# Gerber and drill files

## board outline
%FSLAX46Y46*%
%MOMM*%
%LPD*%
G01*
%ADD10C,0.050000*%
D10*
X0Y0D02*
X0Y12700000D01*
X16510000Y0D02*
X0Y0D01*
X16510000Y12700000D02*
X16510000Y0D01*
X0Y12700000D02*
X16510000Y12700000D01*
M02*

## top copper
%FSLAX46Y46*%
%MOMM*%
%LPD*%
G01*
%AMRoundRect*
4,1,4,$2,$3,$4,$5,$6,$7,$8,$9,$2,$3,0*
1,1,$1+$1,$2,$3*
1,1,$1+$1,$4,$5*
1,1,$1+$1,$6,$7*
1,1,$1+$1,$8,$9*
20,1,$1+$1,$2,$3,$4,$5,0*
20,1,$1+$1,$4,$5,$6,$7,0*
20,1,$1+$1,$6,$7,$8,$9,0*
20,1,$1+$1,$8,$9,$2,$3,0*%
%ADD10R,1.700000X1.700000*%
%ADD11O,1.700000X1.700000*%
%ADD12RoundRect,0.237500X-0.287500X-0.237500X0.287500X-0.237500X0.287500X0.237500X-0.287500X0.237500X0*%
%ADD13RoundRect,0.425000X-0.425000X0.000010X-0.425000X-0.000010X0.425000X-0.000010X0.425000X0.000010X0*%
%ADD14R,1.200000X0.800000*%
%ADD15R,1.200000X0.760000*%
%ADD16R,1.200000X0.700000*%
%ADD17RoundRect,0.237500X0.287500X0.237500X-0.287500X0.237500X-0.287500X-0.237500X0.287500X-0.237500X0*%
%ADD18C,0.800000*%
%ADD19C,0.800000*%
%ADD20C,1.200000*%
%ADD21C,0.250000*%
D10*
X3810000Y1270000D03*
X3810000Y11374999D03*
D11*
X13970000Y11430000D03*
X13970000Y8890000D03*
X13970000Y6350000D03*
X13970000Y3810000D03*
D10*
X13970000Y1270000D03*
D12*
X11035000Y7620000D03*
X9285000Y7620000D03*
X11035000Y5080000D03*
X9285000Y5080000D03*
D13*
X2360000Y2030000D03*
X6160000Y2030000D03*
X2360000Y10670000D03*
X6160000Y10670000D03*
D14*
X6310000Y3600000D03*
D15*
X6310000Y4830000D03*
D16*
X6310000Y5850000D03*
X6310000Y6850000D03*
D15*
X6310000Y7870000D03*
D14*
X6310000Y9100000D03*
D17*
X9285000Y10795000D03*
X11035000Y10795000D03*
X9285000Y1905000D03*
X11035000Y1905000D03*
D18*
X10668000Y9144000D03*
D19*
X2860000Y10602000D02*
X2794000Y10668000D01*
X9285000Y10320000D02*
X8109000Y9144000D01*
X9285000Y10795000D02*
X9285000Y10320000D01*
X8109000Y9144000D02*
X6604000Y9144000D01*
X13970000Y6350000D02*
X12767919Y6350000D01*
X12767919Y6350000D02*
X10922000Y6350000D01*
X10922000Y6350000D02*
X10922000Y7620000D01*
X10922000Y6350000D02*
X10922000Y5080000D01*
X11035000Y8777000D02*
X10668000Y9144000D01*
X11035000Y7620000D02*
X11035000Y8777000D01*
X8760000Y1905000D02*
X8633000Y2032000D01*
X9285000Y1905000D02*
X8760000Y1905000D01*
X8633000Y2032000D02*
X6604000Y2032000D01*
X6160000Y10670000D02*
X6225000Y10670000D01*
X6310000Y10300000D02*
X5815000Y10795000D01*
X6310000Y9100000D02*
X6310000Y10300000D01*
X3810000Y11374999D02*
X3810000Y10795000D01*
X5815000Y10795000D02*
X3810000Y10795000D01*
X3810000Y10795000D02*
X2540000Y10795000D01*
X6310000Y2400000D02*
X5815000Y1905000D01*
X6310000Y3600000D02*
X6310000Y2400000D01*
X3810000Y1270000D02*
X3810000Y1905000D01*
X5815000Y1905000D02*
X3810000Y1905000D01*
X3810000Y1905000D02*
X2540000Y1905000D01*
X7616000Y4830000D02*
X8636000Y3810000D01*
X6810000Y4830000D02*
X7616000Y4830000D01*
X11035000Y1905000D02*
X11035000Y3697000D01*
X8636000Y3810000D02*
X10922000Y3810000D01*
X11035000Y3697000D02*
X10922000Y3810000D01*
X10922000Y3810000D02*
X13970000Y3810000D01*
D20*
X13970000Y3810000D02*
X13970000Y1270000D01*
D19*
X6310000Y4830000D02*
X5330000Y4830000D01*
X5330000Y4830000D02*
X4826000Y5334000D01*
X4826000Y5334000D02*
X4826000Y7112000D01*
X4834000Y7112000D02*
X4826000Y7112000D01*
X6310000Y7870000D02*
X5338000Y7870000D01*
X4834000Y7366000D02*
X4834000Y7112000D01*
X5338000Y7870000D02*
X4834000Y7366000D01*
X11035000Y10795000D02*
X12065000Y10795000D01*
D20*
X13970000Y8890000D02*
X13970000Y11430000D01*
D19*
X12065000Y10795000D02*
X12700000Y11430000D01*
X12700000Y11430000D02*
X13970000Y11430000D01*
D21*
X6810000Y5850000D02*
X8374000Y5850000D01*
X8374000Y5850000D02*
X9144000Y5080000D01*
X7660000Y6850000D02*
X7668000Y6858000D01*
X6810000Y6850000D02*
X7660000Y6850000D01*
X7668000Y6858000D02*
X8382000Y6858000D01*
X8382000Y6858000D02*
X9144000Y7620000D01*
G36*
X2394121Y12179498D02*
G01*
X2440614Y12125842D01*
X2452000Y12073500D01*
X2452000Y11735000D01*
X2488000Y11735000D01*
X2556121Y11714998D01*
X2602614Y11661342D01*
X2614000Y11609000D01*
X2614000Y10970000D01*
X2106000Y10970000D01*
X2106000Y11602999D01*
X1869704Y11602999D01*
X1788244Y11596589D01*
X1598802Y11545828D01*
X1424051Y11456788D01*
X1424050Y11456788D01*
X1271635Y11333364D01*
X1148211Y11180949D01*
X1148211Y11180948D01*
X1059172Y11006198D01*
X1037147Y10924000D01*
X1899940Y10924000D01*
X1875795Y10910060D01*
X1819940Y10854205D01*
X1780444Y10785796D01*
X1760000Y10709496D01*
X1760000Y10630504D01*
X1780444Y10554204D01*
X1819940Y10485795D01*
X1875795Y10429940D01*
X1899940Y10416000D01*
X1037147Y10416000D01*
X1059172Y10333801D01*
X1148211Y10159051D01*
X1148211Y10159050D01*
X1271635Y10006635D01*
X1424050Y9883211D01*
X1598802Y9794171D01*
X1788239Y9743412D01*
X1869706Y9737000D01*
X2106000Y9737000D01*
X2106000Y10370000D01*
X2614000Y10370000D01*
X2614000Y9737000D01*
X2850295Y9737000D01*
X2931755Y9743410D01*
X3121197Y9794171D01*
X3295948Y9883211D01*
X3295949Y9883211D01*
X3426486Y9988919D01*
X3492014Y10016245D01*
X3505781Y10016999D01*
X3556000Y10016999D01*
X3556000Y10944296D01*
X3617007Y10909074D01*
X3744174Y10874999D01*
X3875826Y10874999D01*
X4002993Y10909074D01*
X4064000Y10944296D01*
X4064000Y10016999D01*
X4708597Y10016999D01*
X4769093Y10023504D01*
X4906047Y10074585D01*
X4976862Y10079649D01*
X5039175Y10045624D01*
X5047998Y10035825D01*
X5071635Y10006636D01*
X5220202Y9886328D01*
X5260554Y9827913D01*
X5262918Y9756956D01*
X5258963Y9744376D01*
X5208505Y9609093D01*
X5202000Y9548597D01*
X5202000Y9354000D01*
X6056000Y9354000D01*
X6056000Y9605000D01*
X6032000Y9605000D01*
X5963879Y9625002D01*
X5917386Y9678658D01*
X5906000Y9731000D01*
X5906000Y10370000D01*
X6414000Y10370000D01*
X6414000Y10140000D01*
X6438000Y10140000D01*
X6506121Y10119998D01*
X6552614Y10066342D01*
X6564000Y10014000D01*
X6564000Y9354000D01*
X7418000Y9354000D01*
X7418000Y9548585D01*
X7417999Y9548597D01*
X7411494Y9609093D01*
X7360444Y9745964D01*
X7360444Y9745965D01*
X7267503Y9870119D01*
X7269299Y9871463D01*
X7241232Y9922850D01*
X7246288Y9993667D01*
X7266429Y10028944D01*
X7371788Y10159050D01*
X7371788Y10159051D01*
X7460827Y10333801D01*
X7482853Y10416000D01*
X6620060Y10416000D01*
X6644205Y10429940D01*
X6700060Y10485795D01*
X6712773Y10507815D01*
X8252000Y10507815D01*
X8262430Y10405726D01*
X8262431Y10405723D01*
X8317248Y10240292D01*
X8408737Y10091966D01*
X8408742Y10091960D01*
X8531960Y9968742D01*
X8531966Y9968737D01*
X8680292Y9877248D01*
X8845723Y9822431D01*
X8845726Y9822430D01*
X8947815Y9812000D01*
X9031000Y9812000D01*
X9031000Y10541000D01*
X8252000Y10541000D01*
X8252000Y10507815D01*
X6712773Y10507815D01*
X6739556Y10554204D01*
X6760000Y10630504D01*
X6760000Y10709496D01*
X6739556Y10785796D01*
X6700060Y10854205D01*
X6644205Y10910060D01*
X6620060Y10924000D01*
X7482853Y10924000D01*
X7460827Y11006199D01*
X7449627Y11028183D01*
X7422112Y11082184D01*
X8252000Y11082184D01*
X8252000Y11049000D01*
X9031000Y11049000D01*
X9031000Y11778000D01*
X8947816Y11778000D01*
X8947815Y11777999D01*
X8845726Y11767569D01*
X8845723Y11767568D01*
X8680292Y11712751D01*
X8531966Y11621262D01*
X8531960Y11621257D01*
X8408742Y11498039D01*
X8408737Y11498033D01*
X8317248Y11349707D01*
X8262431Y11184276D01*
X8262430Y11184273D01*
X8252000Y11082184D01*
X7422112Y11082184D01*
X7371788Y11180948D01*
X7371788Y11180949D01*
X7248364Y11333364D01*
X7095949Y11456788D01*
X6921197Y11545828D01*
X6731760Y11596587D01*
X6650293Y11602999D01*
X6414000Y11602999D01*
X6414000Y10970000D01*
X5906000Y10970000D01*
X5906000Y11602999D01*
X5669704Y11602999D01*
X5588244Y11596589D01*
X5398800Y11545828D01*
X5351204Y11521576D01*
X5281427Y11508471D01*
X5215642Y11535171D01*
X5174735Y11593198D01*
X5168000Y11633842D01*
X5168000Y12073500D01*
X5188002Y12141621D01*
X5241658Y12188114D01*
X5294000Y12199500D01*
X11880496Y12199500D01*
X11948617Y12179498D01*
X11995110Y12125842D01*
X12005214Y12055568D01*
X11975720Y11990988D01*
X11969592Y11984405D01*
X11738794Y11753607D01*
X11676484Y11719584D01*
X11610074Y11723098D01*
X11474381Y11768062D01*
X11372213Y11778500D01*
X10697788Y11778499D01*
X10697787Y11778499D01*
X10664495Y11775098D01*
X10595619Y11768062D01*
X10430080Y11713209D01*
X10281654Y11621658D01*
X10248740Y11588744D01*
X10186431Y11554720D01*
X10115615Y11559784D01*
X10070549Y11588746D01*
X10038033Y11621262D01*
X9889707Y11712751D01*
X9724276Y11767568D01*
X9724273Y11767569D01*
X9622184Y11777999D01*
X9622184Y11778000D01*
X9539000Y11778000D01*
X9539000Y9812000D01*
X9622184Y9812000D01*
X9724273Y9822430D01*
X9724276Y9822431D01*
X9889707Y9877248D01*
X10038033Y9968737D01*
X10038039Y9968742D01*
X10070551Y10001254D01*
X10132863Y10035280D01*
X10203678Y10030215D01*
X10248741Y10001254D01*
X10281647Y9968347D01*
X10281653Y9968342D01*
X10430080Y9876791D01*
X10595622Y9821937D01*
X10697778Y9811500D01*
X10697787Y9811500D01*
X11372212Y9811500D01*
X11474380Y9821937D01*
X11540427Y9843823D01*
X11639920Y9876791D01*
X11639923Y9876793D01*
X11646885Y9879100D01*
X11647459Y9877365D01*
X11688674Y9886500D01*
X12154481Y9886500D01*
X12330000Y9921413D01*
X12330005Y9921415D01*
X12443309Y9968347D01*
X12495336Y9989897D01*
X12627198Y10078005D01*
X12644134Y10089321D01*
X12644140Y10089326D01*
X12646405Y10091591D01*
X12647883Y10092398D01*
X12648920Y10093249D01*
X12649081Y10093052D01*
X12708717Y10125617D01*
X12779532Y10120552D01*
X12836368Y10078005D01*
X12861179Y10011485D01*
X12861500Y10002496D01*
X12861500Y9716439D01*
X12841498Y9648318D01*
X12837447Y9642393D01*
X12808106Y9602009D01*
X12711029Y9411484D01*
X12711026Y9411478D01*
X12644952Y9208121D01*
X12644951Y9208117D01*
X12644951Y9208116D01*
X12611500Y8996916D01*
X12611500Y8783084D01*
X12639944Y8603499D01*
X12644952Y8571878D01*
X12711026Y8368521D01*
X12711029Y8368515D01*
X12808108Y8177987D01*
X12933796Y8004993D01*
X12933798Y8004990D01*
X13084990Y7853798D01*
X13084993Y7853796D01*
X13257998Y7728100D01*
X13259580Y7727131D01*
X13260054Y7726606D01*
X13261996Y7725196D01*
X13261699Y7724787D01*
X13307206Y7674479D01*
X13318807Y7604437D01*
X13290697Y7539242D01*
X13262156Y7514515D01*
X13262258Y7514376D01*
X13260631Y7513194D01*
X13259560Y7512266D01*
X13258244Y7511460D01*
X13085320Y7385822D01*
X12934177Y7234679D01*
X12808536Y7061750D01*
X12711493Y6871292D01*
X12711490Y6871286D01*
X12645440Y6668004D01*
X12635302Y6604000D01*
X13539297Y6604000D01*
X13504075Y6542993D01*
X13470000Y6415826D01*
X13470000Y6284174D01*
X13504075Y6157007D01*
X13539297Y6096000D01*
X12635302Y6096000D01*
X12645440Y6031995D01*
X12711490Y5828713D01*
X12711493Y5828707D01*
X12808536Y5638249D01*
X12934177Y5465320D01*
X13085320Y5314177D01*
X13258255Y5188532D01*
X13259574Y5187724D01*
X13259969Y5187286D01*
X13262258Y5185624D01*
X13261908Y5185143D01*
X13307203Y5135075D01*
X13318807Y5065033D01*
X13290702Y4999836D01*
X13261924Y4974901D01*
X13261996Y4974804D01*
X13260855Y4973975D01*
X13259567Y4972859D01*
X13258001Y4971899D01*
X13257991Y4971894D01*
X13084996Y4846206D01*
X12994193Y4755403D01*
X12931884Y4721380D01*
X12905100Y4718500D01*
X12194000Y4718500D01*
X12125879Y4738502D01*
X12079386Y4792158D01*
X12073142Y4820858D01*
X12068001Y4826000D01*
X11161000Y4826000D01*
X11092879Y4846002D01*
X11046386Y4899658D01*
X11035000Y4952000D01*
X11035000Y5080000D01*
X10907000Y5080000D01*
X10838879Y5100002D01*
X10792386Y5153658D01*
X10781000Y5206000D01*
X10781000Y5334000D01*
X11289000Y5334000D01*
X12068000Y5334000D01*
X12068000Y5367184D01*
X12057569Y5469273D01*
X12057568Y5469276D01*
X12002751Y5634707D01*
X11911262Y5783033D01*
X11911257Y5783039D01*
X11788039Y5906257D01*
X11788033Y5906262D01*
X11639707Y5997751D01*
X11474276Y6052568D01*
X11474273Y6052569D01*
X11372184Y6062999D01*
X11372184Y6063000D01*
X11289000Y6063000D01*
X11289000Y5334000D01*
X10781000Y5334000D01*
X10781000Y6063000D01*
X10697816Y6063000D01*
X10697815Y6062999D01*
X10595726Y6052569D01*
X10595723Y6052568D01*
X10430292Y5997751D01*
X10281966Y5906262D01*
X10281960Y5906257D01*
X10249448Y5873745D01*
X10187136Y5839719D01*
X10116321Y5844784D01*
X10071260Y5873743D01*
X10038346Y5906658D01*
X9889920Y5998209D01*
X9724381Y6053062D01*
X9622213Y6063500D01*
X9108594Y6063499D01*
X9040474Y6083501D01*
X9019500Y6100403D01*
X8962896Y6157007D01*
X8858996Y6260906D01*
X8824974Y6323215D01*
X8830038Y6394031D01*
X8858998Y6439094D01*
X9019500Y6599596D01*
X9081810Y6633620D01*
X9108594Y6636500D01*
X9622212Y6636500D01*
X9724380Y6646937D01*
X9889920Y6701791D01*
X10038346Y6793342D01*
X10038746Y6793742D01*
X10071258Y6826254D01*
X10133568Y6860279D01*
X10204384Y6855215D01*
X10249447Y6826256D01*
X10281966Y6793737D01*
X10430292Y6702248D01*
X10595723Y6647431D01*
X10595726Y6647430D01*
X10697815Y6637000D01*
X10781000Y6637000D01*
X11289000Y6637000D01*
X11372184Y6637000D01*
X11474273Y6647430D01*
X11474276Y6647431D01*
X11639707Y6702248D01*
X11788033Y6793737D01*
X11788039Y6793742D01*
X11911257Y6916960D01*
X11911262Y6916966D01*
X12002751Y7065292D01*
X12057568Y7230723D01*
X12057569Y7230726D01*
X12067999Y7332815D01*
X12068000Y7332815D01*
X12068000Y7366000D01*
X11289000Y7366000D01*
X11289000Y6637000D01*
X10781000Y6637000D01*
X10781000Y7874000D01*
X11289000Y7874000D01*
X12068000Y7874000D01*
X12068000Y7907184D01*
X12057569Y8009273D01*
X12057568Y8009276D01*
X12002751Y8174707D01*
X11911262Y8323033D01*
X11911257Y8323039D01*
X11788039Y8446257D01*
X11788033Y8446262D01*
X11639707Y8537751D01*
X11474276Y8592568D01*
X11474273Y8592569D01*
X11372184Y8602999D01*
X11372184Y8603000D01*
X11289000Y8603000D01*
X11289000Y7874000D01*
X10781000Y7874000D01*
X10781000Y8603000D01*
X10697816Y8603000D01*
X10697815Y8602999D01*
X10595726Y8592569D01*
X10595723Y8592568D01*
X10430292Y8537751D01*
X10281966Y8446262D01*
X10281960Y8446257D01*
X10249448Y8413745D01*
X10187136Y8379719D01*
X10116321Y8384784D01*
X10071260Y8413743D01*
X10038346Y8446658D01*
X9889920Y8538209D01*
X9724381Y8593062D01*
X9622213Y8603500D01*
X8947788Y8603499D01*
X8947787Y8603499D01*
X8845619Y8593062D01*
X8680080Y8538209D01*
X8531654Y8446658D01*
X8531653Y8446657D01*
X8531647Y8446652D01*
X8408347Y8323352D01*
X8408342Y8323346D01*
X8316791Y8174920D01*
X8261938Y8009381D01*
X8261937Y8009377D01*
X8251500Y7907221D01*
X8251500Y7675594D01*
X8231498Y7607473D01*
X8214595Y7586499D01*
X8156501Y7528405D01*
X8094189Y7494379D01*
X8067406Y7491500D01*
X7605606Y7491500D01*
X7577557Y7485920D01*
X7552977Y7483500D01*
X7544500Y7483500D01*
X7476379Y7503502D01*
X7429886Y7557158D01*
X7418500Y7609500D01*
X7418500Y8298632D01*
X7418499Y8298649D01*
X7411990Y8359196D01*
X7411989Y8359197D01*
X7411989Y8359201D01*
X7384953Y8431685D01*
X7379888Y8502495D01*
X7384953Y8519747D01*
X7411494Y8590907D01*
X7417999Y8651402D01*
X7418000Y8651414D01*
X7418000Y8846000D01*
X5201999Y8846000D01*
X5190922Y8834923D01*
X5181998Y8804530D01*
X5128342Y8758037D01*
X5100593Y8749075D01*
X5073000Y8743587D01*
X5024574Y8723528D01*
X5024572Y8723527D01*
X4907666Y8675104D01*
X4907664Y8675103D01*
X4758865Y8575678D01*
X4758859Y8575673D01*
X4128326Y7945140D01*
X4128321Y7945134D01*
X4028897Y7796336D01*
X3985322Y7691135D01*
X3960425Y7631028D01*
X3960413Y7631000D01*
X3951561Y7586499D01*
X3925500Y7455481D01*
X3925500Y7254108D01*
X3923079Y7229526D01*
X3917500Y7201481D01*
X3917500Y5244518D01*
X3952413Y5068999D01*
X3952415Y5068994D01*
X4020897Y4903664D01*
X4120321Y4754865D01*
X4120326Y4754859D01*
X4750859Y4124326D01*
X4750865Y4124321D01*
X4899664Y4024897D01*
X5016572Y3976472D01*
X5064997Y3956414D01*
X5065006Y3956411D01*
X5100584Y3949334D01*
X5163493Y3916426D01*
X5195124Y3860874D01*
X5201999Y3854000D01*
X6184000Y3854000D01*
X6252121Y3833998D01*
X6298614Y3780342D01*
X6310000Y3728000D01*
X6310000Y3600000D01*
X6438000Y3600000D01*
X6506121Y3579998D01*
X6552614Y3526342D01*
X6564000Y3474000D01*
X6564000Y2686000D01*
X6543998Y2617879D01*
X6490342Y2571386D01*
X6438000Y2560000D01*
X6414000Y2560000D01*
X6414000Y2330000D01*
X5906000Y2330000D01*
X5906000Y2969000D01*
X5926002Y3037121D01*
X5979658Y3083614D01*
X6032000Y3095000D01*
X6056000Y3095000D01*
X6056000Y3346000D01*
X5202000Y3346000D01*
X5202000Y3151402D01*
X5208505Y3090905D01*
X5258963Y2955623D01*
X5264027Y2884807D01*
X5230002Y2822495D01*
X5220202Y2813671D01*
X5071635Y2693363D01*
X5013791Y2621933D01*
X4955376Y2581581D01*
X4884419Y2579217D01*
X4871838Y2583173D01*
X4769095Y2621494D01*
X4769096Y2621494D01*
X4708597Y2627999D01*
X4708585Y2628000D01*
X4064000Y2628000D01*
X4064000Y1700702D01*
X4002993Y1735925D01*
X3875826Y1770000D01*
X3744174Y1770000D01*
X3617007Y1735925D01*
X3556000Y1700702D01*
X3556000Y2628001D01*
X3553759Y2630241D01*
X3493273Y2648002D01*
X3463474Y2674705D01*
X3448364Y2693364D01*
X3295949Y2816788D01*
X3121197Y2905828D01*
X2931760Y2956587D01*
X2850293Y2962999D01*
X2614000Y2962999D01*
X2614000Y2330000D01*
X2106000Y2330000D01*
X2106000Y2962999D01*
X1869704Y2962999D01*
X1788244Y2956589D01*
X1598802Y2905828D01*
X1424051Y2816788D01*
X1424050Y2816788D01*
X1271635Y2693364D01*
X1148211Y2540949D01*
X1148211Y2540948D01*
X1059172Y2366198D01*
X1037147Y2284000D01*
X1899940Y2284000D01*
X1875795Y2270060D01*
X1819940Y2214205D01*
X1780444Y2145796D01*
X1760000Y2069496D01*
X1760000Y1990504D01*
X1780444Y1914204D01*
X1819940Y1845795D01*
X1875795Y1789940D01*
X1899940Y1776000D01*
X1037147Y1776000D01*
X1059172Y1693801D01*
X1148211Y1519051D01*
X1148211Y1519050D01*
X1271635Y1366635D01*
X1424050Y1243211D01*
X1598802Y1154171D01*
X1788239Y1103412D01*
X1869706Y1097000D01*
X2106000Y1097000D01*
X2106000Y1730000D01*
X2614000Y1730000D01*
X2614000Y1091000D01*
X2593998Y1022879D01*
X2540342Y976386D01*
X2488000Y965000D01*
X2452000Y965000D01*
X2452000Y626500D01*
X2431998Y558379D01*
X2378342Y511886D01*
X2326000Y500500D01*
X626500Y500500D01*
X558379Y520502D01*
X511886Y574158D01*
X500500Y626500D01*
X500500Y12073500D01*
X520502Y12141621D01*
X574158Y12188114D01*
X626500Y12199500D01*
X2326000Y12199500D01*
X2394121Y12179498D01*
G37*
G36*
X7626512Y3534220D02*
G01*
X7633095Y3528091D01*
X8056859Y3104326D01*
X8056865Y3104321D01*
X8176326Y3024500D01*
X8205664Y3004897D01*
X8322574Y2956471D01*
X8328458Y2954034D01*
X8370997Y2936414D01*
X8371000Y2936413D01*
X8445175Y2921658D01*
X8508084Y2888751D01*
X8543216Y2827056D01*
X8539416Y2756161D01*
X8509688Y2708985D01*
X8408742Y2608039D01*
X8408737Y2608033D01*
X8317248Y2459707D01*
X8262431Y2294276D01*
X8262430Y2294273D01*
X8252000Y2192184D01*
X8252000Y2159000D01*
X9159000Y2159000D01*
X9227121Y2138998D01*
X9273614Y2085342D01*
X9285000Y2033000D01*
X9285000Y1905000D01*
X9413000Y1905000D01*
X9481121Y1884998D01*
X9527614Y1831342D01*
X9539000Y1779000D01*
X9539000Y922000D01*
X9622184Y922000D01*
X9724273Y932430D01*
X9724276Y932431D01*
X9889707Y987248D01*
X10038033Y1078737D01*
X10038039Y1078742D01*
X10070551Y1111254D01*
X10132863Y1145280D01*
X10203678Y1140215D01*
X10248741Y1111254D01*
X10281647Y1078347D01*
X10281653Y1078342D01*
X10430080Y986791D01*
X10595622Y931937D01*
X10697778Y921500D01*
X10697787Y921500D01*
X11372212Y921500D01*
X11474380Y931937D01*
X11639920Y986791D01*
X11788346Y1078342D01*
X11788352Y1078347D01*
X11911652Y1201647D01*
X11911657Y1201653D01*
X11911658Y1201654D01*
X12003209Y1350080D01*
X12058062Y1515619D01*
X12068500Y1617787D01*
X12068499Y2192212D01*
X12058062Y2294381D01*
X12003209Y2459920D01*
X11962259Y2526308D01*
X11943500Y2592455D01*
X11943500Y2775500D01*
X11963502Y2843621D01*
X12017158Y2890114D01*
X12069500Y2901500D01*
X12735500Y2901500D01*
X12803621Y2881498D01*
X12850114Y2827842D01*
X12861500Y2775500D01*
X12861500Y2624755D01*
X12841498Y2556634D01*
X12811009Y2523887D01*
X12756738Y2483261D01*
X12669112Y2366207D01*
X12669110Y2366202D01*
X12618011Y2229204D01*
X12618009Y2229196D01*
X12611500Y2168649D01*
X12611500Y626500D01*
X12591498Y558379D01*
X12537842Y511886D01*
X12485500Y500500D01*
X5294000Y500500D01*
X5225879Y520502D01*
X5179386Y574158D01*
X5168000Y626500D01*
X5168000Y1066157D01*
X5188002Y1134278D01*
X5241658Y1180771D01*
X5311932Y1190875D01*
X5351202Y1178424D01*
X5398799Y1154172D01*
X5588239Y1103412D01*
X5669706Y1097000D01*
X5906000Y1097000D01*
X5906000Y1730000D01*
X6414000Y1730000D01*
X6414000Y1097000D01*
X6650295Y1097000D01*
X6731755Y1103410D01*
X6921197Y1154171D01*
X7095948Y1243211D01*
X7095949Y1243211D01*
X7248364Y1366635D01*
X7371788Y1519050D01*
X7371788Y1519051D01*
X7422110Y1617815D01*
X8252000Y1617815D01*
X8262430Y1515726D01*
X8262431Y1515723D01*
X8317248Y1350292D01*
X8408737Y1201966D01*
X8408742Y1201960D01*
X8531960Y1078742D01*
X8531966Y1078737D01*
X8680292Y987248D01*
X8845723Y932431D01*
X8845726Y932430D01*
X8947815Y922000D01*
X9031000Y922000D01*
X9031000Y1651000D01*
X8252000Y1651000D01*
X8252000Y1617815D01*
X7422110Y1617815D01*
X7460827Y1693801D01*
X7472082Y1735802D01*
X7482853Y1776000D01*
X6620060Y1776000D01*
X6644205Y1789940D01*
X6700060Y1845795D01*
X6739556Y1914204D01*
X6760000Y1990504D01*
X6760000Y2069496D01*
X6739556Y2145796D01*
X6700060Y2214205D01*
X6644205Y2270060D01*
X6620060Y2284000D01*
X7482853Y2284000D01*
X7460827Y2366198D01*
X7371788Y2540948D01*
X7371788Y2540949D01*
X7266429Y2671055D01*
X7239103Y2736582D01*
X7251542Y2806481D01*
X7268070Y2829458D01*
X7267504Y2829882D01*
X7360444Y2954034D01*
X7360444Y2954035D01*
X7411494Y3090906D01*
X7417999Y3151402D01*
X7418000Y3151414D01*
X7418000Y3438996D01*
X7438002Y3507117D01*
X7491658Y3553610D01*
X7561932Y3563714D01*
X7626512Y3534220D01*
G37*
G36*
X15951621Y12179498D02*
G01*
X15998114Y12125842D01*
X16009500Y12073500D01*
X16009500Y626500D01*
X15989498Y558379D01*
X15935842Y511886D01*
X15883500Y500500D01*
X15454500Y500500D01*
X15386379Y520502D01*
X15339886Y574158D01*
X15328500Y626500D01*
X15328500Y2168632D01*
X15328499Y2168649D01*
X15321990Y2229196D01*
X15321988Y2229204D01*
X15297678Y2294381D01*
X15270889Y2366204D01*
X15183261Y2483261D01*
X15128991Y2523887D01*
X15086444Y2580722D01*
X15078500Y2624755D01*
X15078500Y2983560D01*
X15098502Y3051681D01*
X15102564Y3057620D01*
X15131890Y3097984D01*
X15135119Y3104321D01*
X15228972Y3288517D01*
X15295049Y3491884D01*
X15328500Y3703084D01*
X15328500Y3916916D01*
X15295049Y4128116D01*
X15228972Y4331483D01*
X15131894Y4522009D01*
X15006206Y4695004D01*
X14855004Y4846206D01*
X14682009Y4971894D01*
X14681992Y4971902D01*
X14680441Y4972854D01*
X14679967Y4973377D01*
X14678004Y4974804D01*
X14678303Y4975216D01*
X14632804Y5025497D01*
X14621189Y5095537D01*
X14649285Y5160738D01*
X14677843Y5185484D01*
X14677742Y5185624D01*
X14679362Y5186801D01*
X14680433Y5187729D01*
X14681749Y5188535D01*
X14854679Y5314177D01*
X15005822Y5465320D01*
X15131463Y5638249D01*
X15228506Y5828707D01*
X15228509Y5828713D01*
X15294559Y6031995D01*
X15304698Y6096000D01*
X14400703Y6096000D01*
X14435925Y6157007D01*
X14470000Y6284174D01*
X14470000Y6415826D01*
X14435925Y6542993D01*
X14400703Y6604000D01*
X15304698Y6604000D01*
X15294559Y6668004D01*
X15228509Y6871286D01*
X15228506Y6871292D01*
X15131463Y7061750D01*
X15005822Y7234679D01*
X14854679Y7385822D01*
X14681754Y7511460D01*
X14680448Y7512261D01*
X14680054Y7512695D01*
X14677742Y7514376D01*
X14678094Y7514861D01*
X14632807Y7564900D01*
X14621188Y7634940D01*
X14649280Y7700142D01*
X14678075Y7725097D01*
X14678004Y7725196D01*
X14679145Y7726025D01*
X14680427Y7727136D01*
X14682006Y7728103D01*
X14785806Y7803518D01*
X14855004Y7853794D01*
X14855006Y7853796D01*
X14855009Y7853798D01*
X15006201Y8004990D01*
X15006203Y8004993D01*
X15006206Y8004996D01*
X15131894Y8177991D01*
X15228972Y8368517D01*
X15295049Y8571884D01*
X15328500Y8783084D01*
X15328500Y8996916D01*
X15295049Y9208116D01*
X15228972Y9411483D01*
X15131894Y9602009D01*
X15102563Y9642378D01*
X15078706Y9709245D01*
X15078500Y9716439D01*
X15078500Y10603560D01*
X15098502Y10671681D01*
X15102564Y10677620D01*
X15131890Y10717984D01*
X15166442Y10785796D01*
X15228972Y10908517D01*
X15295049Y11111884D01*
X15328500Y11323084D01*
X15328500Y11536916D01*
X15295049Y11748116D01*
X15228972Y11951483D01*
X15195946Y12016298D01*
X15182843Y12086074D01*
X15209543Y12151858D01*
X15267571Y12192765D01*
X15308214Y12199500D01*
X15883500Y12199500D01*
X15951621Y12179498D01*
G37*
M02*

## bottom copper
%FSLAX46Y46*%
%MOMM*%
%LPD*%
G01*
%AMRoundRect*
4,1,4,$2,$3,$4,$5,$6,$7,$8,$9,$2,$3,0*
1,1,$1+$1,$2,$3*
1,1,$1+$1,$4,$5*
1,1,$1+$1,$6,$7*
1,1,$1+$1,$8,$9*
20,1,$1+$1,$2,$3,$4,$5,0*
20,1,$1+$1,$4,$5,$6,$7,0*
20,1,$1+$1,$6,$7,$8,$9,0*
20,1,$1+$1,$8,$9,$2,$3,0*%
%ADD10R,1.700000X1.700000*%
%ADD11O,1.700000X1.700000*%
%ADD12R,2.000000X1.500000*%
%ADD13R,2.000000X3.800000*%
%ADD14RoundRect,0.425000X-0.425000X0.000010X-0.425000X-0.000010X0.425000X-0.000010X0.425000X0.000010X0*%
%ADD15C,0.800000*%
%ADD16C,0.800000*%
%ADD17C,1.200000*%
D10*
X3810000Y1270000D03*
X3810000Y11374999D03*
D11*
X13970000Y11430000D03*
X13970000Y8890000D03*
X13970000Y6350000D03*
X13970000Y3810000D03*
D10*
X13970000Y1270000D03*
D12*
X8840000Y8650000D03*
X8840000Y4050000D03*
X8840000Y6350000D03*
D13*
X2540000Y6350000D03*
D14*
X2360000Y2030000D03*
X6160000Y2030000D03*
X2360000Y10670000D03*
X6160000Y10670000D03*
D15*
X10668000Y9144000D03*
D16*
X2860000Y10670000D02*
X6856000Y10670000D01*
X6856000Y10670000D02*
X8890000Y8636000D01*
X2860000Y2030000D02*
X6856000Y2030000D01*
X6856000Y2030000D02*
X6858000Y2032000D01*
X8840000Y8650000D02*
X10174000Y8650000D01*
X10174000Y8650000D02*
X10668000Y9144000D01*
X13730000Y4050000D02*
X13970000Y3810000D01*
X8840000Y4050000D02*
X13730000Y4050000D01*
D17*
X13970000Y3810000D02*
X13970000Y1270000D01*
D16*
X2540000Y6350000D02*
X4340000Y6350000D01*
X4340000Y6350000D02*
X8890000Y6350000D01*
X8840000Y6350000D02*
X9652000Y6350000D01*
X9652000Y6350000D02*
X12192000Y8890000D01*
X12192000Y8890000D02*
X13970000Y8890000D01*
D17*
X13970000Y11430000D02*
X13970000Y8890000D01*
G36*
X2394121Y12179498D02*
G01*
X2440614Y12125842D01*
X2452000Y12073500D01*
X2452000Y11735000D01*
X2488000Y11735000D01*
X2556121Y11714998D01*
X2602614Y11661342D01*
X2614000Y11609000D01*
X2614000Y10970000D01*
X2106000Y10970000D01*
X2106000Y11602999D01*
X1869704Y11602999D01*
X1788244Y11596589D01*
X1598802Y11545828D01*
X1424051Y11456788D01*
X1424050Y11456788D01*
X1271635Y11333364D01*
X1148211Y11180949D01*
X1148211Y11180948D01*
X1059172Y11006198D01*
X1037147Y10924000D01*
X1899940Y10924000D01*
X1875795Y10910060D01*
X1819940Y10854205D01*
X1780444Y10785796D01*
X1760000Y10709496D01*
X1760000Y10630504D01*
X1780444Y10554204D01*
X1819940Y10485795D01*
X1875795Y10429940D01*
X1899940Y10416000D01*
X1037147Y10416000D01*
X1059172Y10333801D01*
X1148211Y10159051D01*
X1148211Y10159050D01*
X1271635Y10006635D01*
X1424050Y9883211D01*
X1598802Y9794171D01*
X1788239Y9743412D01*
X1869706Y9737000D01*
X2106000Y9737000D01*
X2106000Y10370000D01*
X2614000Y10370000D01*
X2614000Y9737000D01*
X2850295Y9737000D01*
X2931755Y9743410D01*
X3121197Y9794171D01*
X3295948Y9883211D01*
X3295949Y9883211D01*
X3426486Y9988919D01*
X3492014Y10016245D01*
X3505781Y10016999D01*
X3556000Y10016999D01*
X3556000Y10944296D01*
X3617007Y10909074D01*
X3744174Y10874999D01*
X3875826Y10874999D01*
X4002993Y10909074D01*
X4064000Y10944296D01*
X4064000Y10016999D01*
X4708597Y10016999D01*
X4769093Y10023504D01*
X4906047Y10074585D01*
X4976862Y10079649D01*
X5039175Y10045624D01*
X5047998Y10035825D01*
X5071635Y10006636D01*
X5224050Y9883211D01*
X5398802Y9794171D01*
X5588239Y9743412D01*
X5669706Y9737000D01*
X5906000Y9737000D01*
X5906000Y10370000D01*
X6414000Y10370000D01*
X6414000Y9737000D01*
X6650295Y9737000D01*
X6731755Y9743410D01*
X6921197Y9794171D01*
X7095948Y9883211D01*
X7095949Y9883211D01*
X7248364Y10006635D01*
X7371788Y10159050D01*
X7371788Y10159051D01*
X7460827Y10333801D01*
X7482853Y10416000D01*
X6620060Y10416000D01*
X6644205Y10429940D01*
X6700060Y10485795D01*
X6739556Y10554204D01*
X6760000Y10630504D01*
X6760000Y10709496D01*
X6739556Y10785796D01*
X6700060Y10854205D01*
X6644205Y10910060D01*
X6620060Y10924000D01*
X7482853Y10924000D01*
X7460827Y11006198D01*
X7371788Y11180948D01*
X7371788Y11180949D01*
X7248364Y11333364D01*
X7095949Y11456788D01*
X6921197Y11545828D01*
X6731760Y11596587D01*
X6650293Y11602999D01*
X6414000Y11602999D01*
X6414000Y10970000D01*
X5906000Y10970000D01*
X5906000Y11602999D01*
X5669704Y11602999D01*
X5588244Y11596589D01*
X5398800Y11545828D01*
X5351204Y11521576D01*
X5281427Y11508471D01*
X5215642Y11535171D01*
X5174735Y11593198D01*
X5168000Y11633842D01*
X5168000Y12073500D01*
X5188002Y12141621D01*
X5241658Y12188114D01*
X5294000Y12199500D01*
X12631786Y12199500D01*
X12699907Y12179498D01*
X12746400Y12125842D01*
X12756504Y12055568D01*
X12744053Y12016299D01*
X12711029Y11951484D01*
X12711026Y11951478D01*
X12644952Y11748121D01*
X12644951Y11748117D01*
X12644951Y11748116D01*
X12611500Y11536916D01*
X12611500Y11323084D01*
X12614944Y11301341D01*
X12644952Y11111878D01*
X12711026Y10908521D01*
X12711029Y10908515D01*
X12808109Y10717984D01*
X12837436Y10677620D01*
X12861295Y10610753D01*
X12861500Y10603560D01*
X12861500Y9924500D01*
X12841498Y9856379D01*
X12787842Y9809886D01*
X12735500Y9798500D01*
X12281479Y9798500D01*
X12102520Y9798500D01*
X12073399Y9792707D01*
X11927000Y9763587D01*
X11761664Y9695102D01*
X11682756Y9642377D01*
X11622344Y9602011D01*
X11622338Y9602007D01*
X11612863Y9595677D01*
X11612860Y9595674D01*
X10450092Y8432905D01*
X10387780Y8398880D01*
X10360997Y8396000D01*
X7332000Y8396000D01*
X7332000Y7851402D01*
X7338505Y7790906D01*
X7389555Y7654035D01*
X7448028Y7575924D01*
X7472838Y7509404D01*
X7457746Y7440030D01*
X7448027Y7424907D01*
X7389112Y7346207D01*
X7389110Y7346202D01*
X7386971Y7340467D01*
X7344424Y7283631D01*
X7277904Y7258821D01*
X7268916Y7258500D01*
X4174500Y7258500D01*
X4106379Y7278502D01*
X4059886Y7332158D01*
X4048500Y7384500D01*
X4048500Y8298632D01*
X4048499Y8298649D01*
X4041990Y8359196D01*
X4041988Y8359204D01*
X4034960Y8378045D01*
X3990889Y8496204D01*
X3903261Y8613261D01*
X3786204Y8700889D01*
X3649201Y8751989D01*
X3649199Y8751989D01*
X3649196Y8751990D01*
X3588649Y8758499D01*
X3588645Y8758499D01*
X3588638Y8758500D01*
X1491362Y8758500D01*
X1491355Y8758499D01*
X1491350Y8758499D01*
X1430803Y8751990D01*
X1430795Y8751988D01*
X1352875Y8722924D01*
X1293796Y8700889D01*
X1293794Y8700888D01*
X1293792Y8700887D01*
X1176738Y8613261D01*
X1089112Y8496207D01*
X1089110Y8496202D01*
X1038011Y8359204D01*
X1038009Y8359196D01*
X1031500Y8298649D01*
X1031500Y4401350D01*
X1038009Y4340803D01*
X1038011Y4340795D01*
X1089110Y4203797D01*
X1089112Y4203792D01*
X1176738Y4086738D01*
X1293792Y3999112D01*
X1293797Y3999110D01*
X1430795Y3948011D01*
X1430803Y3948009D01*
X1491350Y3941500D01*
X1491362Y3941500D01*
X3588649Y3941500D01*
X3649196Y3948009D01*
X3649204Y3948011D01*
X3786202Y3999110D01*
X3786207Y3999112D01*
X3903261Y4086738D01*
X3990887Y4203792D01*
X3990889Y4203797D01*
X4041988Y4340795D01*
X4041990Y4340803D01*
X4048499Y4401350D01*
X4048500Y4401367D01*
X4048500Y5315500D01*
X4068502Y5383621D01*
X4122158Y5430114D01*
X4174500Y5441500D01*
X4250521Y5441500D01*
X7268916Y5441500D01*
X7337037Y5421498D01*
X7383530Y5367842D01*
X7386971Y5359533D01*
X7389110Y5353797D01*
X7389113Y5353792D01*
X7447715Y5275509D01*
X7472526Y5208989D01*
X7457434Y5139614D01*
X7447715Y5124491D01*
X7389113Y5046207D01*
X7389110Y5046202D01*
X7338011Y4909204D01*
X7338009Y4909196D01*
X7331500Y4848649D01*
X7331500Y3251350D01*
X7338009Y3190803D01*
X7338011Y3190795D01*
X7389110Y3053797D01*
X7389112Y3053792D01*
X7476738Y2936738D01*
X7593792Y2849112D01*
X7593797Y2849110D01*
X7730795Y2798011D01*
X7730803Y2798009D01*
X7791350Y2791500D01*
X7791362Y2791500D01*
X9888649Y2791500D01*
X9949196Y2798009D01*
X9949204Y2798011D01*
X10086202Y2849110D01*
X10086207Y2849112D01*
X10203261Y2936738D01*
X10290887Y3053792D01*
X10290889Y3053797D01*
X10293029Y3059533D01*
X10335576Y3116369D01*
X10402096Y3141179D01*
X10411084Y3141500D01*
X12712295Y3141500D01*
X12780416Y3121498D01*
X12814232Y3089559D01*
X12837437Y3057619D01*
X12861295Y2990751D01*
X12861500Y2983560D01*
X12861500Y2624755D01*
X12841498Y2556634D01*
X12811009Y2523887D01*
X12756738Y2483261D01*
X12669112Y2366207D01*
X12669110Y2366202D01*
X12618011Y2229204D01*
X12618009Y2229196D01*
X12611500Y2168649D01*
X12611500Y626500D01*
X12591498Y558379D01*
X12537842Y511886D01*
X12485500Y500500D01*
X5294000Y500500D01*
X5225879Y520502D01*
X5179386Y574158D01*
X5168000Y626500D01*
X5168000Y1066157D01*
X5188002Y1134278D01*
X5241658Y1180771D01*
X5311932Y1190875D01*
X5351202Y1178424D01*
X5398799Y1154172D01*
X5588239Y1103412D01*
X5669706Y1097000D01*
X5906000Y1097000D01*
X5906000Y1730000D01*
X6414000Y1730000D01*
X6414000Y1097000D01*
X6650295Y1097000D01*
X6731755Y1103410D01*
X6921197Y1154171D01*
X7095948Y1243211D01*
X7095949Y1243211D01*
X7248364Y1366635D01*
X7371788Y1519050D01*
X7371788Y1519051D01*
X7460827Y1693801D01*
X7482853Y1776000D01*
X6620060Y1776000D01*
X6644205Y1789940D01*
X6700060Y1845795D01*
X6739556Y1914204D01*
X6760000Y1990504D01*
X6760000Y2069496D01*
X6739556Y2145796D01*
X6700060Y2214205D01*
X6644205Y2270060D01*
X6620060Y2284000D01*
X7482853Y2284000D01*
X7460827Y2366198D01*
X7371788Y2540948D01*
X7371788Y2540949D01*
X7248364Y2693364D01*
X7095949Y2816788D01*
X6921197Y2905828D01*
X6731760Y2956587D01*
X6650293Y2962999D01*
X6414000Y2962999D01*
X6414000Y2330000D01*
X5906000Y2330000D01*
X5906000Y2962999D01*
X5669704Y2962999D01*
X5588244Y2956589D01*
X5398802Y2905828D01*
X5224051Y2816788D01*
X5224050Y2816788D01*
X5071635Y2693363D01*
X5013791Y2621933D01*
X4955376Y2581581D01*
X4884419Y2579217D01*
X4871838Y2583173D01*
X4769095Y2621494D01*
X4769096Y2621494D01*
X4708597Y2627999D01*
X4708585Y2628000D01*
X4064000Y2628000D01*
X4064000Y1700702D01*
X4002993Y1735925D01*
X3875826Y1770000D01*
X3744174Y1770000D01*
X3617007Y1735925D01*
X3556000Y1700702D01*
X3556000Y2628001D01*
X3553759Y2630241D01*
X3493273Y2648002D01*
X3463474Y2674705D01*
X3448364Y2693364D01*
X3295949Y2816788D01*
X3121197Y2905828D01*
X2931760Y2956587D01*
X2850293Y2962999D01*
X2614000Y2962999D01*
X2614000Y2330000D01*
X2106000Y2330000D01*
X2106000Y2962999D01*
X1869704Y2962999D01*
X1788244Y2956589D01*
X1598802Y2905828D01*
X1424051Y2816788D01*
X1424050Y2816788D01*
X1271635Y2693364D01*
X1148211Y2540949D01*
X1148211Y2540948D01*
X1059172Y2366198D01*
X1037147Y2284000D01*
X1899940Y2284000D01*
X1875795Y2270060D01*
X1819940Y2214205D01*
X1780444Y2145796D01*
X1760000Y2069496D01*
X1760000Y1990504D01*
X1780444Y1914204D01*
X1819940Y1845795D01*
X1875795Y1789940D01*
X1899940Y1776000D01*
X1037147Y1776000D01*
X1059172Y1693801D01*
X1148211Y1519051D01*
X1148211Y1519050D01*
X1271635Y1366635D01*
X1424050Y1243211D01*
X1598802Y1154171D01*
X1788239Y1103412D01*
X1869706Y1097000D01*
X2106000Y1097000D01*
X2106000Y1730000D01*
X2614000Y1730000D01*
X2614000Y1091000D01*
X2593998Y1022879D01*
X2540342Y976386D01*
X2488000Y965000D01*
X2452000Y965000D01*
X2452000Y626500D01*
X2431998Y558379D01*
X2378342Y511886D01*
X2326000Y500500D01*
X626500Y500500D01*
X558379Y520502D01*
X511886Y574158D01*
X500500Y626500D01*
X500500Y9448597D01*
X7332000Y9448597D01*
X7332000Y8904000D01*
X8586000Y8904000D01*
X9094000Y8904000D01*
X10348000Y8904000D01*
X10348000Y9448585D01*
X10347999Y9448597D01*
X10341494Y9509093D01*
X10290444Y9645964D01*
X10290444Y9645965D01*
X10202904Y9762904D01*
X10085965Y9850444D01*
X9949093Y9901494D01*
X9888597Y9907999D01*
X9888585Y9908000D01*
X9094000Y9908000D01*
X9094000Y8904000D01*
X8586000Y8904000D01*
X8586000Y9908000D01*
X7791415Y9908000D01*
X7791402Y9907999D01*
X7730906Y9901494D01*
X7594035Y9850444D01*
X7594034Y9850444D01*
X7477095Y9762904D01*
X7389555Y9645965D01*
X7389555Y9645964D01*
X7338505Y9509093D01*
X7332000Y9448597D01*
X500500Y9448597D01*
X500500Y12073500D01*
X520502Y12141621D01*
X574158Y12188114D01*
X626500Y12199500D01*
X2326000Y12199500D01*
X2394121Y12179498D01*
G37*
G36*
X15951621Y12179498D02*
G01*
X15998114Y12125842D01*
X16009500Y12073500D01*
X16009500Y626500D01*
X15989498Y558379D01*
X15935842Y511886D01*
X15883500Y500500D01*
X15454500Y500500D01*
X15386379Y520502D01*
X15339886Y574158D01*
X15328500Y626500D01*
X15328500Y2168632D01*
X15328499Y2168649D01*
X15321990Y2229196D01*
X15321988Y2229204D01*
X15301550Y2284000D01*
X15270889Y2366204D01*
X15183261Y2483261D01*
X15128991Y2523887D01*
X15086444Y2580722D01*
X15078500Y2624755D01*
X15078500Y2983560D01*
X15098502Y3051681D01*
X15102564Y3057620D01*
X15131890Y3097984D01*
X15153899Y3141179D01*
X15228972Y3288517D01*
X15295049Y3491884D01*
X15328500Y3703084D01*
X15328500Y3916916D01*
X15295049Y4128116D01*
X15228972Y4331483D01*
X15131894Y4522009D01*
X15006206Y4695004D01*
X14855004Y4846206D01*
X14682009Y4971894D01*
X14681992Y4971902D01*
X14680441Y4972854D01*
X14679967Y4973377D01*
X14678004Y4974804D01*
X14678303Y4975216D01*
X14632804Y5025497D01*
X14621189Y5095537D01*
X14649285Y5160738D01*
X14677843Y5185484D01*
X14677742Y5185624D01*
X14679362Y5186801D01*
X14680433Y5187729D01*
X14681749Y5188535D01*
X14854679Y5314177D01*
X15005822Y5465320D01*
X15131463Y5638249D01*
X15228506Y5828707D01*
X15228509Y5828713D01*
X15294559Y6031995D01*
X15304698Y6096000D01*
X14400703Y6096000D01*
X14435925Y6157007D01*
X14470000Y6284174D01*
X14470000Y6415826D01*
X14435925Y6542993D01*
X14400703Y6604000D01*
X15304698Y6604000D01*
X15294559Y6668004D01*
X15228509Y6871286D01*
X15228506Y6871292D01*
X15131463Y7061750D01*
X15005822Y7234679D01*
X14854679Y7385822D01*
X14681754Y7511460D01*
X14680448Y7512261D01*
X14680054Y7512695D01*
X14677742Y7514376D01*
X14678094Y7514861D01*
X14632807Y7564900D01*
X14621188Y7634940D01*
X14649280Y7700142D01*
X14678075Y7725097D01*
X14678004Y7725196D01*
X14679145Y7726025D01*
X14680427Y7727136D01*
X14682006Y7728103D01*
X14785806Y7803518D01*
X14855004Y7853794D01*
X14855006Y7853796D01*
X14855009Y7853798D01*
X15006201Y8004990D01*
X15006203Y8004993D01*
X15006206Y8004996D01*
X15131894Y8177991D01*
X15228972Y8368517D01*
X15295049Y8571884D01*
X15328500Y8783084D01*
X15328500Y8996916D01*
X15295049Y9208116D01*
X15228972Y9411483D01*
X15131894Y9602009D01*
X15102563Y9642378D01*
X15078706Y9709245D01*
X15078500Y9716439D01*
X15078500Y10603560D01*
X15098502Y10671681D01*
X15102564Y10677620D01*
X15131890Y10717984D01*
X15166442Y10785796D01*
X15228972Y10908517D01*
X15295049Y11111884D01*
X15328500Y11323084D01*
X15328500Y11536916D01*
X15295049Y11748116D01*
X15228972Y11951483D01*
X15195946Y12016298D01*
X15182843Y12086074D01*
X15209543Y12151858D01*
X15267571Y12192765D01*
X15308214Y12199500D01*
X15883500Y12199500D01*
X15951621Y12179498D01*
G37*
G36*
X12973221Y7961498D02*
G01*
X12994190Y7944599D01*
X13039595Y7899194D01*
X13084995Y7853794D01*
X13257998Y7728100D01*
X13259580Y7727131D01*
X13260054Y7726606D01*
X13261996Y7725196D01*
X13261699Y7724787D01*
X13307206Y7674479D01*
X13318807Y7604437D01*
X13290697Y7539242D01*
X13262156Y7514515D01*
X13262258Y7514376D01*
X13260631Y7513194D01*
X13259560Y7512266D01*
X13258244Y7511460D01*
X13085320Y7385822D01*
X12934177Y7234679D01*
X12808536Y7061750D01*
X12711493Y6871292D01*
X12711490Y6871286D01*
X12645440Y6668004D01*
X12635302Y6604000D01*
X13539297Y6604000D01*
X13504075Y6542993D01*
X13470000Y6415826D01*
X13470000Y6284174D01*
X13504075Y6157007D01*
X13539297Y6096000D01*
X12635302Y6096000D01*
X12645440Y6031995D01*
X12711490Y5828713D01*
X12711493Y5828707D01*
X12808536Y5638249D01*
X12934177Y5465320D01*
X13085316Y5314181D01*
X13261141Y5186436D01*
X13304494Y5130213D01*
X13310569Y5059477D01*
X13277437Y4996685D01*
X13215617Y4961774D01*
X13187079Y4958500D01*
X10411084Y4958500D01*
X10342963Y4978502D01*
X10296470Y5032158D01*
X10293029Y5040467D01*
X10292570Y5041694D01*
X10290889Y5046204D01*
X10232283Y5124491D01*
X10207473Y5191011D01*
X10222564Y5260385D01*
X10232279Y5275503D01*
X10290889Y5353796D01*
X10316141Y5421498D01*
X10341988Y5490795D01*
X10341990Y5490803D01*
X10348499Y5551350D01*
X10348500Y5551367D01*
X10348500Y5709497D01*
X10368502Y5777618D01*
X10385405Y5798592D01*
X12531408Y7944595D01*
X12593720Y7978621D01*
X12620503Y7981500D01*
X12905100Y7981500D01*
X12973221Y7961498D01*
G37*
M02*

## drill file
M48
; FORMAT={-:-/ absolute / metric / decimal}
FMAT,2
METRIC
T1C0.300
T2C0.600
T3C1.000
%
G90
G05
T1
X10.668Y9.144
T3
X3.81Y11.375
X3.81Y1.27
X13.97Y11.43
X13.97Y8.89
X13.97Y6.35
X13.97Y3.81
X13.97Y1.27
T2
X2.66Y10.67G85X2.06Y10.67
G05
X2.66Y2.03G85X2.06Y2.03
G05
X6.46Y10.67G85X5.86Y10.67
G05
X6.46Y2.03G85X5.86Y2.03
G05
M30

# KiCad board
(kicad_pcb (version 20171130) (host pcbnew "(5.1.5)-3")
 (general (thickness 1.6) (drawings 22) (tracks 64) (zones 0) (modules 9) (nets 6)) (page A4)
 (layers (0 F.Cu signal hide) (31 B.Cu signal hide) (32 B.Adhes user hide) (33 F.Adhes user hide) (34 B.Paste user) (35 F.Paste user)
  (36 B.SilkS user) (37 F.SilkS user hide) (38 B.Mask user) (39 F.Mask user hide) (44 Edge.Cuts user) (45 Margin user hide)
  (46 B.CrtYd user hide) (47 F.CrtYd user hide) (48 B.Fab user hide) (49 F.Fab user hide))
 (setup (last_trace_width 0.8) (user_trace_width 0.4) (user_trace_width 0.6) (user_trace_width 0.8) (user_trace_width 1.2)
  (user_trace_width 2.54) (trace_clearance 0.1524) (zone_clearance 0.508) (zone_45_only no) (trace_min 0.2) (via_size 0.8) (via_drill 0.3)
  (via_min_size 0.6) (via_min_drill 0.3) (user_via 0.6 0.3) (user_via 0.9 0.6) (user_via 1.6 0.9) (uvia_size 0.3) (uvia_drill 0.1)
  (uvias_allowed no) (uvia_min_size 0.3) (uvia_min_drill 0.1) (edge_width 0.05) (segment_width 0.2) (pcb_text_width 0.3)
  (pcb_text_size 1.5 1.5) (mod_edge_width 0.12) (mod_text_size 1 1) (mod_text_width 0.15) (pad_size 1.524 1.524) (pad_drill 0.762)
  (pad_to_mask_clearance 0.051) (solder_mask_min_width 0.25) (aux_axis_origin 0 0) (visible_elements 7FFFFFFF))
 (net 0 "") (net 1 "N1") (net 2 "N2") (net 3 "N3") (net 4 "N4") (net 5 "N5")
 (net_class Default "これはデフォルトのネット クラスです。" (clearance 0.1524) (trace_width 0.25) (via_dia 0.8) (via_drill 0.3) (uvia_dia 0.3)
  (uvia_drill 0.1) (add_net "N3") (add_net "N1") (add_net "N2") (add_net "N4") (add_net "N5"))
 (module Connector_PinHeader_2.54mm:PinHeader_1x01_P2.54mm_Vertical (layer F.Cu) (at 3.81 -1.27 180)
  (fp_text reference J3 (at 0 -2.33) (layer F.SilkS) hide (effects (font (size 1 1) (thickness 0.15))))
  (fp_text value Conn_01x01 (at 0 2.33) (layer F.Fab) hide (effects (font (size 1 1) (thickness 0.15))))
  (pad 1 thru_hole rect (at 0 0 180) (size 1.7 1.7) (drill 1) (layers *.Cu *.Mask) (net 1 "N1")))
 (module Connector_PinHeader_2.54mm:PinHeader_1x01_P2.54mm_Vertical (layer F.Cu) (at 3.81 -11.374999)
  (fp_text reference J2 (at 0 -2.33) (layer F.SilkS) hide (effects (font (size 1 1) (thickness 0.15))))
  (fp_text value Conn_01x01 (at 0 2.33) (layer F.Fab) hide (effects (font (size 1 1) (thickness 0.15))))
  (pad 1 thru_hole rect (at 0 0) (size 1.7 1.7) (drill 1) (layers *.Cu *.Mask) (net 1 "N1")))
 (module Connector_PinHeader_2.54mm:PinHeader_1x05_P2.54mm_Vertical (layer F.Cu) (at 13.97 -1.27 180)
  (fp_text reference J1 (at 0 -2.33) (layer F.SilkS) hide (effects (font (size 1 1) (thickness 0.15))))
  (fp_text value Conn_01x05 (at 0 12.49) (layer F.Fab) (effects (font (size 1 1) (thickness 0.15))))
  (pad 5 thru_hole oval (at 0 10.16 180) (size 1.7 1.7) (drill 1) (layers *.Cu *.Mask) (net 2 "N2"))
  (pad 4 thru_hole oval (at 0 7.62 180) (size 1.7 1.7) (drill 1) (layers *.Cu *.Mask) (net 2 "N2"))
  (pad 3 thru_hole oval (at 0 5.08 180) (size 1.7 1.7) (drill 1) (layers *.Cu *.Mask) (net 1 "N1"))
  (pad 2 thru_hole oval (at 0 2.54 180) (size 1.7 1.7) (drill 1) (layers *.Cu *.Mask) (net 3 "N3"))
  (pad 1 thru_hole rect (at 0 0 180) (size 1.7 1.7) (drill 1) (layers *.Cu *.Mask) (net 3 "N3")))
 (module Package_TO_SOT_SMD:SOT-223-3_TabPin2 (layer B.Cu) (at 5.69 -6.35 180)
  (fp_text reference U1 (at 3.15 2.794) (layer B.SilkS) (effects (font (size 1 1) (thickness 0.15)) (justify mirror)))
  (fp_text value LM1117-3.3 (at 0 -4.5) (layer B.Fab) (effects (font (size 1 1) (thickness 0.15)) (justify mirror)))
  (pad 1 smd rect (at -3.15 2.3 180) (size 2 1.5) (layers B.Cu B.Paste B.Mask) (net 1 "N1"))
  (pad 3 smd rect (at -3.15 -2.3 180) (size 2 1.5) (layers B.Cu B.Paste B.Mask) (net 3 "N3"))
  (pad 2 smd rect (at -3.15 0 180) (size 2 1.5) (layers B.Cu B.Paste B.Mask) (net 2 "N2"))
  (pad 2 smd rect (at 3.15 0 180) (size 2 3.8) (layers B.Cu B.Paste B.Mask) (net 2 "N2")))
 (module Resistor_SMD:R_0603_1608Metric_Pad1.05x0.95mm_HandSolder (layer F.Cu) (at 10.16 -7.62)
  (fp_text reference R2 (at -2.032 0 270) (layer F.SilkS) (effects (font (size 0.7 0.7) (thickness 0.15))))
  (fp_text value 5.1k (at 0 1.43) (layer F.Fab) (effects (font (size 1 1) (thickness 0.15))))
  (pad 2 smd roundrect (at 0.875 0) (size 1.05 0.95) (layers F.Cu F.Paste F.Mask) (roundrect_rratio 0.25) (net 1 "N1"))
  (pad 1 smd roundrect (at -0.875 0) (size 1.05 0.95) (layers F.Cu F.Paste F.Mask) (roundrect_rratio 0.25) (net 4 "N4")))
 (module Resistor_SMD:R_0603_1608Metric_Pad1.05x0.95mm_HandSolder (layer F.Cu) (at 10.16 -5.08)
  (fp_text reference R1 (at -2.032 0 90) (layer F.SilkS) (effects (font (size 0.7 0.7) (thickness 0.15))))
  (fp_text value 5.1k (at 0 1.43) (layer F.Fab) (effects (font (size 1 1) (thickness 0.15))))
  (pad 2 smd roundrect (at 0.875 0) (size 1.05 0.95) (layers F.Cu F.Paste F.Mask) (roundrect_rratio 0.25) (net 1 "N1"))
  (pad 1 smd roundrect (at -0.875 0) (size 1.05 0.95) (layers F.Cu F.Paste F.Mask) (roundrect_rratio 0.25) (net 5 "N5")))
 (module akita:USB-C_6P (layer F.Cu) (at 3.31 -6.35 270)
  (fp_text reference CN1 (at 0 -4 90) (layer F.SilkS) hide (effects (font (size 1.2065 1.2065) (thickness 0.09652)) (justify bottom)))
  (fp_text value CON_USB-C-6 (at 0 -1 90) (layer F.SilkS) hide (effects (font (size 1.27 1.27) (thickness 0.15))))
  (pad FG thru_hole roundrect (at 4.32 0.95 270) (size 0.85 1.7) (drill oval 0.6 1.2) (layers *.Cu *.Mask) (roundrect_rratio 0.5)
   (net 1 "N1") (solder_mask_margin 0.1016))
  (pad FG thru_hole roundrect (at 4.32 -2.85 270) (size 0.85 1.7) (drill oval 0.6 1.2) (layers *.Cu *.Mask) (roundrect_rratio 0.5)
   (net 1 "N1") (solder_mask_margin 0.1016))
  (pad FG thru_hole roundrect (at -4.32 0.95 270) (size 0.85 1.7) (drill oval 0.6 1.2) (layers *.Cu *.Mask) (roundrect_rratio 0.5)
   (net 1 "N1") (solder_mask_margin 0.1016))
  (pad FG thru_hole roundrect (at -4.32 -2.85 270) (size 0.85 1.7) (drill oval 0.6 1.2) (layers *.Cu *.Mask) (roundrect_rratio 0.5)
   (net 1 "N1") (solder_mask_margin 0.1016))
  (pad A12 smd rect (at 2.75 -3 270) (size 0.8 1.2) (layers F.Cu F.Paste F.Mask) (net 1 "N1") (solder_mask_margin 0.1016))
  (pad A9 smd rect (at 1.52 -3 270) (size 0.76 1.2) (layers F.Cu F.Paste F.Mask) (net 3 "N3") (solder_mask_margin 0.1016))
  (pad B5 smd rect (at 0.5 -3 270) (size 0.7 1.2) (layers F.Cu F.Paste F.Mask) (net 5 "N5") (solder_mask_margin 0.1016))
  (pad A5 smd rect (at -0.5 -3 270) (size 0.7 1.2) (layers F.Cu F.Paste F.Mask) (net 4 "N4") (solder_mask_margin 0.1016))
  (pad B9 smd rect (at -1.52 -3 270) (size 0.76 1.2) (layers F.Cu F.Paste F.Mask) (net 3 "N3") (solder_mask_margin 0.1016))
  (pad B12 smd rect (at -2.75 -3 270) (size 0.8 1.2) (layers F.Cu F.Paste F.Mask) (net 1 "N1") (solder_mask_margin 0.1016)))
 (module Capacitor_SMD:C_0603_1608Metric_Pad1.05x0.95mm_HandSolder (layer F.Cu) (at 10.16 -10.795 180)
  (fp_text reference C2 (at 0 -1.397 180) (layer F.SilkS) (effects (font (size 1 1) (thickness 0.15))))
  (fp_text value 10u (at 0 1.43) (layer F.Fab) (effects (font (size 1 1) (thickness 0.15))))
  (pad 2 smd roundrect (at 0.875 0 180) (size 1.05 0.95) (layers F.Cu F.Paste F.Mask) (roundrect_rratio 0.25) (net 1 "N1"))
  (pad 1 smd roundrect (at -0.875 0 180) (size 1.05 0.95) (layers F.Cu F.Paste F.Mask) (roundrect_rratio 0.25) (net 2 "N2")))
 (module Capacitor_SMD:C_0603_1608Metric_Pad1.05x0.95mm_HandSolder (layer F.Cu) (at 10.16 -1.905 180)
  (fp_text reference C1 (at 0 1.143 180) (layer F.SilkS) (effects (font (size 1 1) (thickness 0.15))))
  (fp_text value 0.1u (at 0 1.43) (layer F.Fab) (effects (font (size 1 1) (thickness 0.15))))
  (pad 2 smd roundrect (at 0.875 0 180) (size 1.05 0.95) (layers F.Cu F.Paste F.Mask) (roundrect_rratio 0.25) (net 1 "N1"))
  (pad 1 smd roundrect (at -0.875 0 180) (size 1.05 0.95) (layers F.Cu F.Paste F.Mask) (roundrect_rratio 0.25) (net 3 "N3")))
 (gr_line (start 0 0) (end 0 -12.7) (layer Edge.Cuts) (width 0.05))
 (gr_line (start 16.51 0) (end 0 0) (layer Edge.Cuts) (width 0.05))
 (gr_line (start 16.51 -12.7) (end 16.51 0) (layer Edge.Cuts) (width 0.05))
 (gr_line (start 0 -12.7) (end 16.51 -12.7) (layer Edge.Cuts) (width 0.05))
 (segment (start 2.86 -10.67) (end 6.856 -10.67) (width 0.8) (layer B.Cu) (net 1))
 (segment (start 6.856 -10.67) (end 8.89 -8.636) (width 0.8) (layer B.Cu) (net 1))
 (segment (start 2.86 -2.03) (end 6.856 -2.03) (width 0.8) (layer B.Cu) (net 1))
 (segment (start 6.856 -2.03) (end 6.858 -2.032) (width 0.8) (layer B.Cu) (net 1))
 (segment (start 2.86 -10.602) (end 2.794 -10.668) (width 0.8) (layer F.Cu) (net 1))
 (segment (start 9.285 -10.32) (end 8.109 -9.144) (width 0.8) (layer F.Cu) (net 1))
 (segment (start 9.285 -10.795) (end 9.285 -10.32) (width 0.8) (layer F.Cu) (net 1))
 (segment (start 8.109 -9.144) (end 6.604 -9.144) (width 0.8) (layer F.Cu) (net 1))
 (segment (start 13.97 -6.35) (end 12.767919 -6.35) (width 0.8) (layer F.Cu) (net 1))
 (segment (start 12.767919 -6.35) (end 10.922 -6.35) (width 0.8) (layer F.Cu) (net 1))
 (segment (start 10.922 -6.35) (end 10.922 -7.62) (width 0.8) (layer F.Cu) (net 1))
 (segment (start 10.922 -6.35) (end 10.922 -5.08) (width 0.8) (layer F.Cu) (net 1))
 (segment (start 8.84 -8.65) (end 10.174 -8.65) (width 0.8) (layer B.Cu) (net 1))
 (via (at 10.668 -9.144) (size 0.8) (drill 0.3) (layers F.Cu B.Cu) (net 1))
 (segment (start 10.174 -8.65) (end 10.668 -9.144) (width 0.8) (layer B.Cu) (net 1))
 (segment (start 11.035 -8.777) (end 10.668 -9.144) (width 0.8) (layer F.Cu) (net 1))
 (segment (start 11.035 -7.62) (end 11.035 -8.777) (width 0.8) (layer F.Cu) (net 1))
 (segment (start 8.76 -1.905) (end 8.633 -2.032) (width 0.8) (layer F.Cu) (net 1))
 (segment (start 9.285 -1.905) (end 8.76 -1.905) (width 0.8) (layer F.Cu) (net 1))
 (segment (start 8.633 -2.032) (end 6.604 -2.032) (width 0.8) (layer F.Cu) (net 1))
 (segment (start 6.16 -10.67) (end 6.225 -10.67) (width 0.8) (layer F.Cu) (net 1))
 (segment (start 6.31 -10.3) (end 5.815 -10.795) (width 0.8) (layer F.Cu) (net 1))
 (segment (start 6.31 -9.1) (end 6.31 -10.3) (width 0.8) (layer F.Cu) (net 1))
 (segment (start 3.81 -11.374999) (end 3.81 -10.795) (width 0.8) (layer F.Cu) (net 1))
 (segment (start 5.815 -10.795) (end 3.81 -10.795) (width 0.8) (layer F.Cu) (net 1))
 (segment (start 3.81 -10.795) (end 2.54 -10.795) (width 0.8) (layer F.Cu) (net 1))
 (segment (start 6.31 -2.4) (end 5.815 -1.905) (width 0.8) (layer F.Cu) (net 1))
 (segment (start 6.31 -3.6) (end 6.31 -2.4) (width 0.8) (layer F.Cu) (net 1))
 (segment (start 3.81 -1.27) (end 3.81 -1.905) (width 0.8) (layer F.Cu) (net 1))
 (segment (start 5.815 -1.905) (end 3.81 -1.905) (width 0.8) (layer F.Cu) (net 1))
 (segment (start 3.81 -1.905) (end 2.54 -1.905) (width 0.8) (layer F.Cu) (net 1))
 (segment (start 13.73 -4.05) (end 13.97 -3.81) (width 0.8) (layer B.Cu) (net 3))
 (segment (start 8.84 -4.05) (end 13.73 -4.05) (width 0.8) (layer B.Cu) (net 3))
 (segment (start 7.616 -4.83) (end 8.636 -3.81) (width 0.8) (layer F.Cu) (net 3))
 (segment (start 6.81 -4.83) (end 7.616 -4.83) (width 0.8) (layer F.Cu) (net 3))
 (segment (start 11.035 -1.905) (end 11.035 -3.697) (width 0.8) (layer F.Cu) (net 3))
 (segment (start 8.636 -3.81) (end 10.922 -3.81) (width 0.8) (layer F.Cu) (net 3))
 (segment (start 11.035 -3.697) (end 10.922 -3.81) (width 0.8) (layer F.Cu) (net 3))
 (segment (start 10.922 -3.81) (end 13.97 -3.81) (width 0.8) (layer F.Cu) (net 3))
 (segment (start 13.97 -3.81) (end 13.97 -1.27) (width 1.2) (layer F.Cu) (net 3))
 (segment (start 13.97 -3.81) (end 13.97 -1.27) (width 1.2) (layer B.Cu) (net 3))
 (segment (start 6.31 -4.83) (end 5.33 -4.83) (width 0.8) (layer F.Cu) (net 3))
 (segment (start 5.33 -4.83) (end 4.826 -5.334) (width 0.8) (layer F.Cu) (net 3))
 (segment (start 4.826 -5.334) (end 4.826 -7.112) (width 0.8) (layer F.Cu) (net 3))
 (segment (start 4.834 -7.112) (end 4.826 -7.112) (width 0.8) (layer F.Cu) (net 3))
 (segment (start 6.31 -7.87) (end 5.338 -7.87) (width 0.8) (layer F.Cu) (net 3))
 (segment (start 4.834 -7.366) (end 4.834 -7.112) (width 0.8) (layer F.Cu) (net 3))
 (segment (start 5.338 -7.87) (end 4.834 -7.366) (width 0.8) (layer F.Cu) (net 3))
 (segment (start 2.54 -6.35) (end 4.34 -6.35) (width 0.8) (layer B.Cu) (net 2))
 (segment (start 4.34 -6.35) (end 8.89 -6.35) (width 0.8) (layer B.Cu) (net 2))
 (segment (start 8.84 -6.35) (end 9.652 -6.35) (width 0.8) (layer B.Cu) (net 2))
 (segment (start 9.652 -6.35) (end 12.192 -8.89) (width 0.8) (layer B.Cu) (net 2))
 (segment (start 12.192 -8.89) (end 13.97 -8.89) (width 0.8) (layer B.Cu) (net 2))
 (segment (start 11.035 -10.795) (end 12.065 -10.795) (width 0.8) (layer F.Cu) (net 2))
 (segment (start 13.97 -8.89) (end 13.97 -11.43) (width 1.2) (layer F.Cu) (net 2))
 (segment (start 12.065 -10.795) (end 12.7 -11.43) (width 0.8) (layer F.Cu) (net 2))
 (segment (start 12.7 -11.43) (end 13.97 -11.43) (width 0.8) (layer F.Cu) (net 2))
 (segment (start 13.97 -11.43) (end 13.97 -8.89) (width 1.2) (layer B.Cu) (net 2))
 (segment (start 6.81 -5.85) (end 8.374 -5.85) (width 0.25) (layer F.Cu) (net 5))
 (segment (start 8.374 -5.85) (end 9.144 -5.08) (width 0.25) (layer F.Cu) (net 5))
 (segment (start 7.66 -6.85) (end 7.668 -6.858) (width 0.25) (layer F.Cu) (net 4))
 (segment (start 6.81 -6.85) (end 7.66 -6.85) (width 0.25) (layer F.Cu) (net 4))
 (segment (start 7.668 -6.858) (end 8.382 -6.858) (width 0.25) (layer F.Cu) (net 4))
 (segment (start 8.382 -6.858) (end 9.144 -7.62) (width 0.25) (layer F.Cu) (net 4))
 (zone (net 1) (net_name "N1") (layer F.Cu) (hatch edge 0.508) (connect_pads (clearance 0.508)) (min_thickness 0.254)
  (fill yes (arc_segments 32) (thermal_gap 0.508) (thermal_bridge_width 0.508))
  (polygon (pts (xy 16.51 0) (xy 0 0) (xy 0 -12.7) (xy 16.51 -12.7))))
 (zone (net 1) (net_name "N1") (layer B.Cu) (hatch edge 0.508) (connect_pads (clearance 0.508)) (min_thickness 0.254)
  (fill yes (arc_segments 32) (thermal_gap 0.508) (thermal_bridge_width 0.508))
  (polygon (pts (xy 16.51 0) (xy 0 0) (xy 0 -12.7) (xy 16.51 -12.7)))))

